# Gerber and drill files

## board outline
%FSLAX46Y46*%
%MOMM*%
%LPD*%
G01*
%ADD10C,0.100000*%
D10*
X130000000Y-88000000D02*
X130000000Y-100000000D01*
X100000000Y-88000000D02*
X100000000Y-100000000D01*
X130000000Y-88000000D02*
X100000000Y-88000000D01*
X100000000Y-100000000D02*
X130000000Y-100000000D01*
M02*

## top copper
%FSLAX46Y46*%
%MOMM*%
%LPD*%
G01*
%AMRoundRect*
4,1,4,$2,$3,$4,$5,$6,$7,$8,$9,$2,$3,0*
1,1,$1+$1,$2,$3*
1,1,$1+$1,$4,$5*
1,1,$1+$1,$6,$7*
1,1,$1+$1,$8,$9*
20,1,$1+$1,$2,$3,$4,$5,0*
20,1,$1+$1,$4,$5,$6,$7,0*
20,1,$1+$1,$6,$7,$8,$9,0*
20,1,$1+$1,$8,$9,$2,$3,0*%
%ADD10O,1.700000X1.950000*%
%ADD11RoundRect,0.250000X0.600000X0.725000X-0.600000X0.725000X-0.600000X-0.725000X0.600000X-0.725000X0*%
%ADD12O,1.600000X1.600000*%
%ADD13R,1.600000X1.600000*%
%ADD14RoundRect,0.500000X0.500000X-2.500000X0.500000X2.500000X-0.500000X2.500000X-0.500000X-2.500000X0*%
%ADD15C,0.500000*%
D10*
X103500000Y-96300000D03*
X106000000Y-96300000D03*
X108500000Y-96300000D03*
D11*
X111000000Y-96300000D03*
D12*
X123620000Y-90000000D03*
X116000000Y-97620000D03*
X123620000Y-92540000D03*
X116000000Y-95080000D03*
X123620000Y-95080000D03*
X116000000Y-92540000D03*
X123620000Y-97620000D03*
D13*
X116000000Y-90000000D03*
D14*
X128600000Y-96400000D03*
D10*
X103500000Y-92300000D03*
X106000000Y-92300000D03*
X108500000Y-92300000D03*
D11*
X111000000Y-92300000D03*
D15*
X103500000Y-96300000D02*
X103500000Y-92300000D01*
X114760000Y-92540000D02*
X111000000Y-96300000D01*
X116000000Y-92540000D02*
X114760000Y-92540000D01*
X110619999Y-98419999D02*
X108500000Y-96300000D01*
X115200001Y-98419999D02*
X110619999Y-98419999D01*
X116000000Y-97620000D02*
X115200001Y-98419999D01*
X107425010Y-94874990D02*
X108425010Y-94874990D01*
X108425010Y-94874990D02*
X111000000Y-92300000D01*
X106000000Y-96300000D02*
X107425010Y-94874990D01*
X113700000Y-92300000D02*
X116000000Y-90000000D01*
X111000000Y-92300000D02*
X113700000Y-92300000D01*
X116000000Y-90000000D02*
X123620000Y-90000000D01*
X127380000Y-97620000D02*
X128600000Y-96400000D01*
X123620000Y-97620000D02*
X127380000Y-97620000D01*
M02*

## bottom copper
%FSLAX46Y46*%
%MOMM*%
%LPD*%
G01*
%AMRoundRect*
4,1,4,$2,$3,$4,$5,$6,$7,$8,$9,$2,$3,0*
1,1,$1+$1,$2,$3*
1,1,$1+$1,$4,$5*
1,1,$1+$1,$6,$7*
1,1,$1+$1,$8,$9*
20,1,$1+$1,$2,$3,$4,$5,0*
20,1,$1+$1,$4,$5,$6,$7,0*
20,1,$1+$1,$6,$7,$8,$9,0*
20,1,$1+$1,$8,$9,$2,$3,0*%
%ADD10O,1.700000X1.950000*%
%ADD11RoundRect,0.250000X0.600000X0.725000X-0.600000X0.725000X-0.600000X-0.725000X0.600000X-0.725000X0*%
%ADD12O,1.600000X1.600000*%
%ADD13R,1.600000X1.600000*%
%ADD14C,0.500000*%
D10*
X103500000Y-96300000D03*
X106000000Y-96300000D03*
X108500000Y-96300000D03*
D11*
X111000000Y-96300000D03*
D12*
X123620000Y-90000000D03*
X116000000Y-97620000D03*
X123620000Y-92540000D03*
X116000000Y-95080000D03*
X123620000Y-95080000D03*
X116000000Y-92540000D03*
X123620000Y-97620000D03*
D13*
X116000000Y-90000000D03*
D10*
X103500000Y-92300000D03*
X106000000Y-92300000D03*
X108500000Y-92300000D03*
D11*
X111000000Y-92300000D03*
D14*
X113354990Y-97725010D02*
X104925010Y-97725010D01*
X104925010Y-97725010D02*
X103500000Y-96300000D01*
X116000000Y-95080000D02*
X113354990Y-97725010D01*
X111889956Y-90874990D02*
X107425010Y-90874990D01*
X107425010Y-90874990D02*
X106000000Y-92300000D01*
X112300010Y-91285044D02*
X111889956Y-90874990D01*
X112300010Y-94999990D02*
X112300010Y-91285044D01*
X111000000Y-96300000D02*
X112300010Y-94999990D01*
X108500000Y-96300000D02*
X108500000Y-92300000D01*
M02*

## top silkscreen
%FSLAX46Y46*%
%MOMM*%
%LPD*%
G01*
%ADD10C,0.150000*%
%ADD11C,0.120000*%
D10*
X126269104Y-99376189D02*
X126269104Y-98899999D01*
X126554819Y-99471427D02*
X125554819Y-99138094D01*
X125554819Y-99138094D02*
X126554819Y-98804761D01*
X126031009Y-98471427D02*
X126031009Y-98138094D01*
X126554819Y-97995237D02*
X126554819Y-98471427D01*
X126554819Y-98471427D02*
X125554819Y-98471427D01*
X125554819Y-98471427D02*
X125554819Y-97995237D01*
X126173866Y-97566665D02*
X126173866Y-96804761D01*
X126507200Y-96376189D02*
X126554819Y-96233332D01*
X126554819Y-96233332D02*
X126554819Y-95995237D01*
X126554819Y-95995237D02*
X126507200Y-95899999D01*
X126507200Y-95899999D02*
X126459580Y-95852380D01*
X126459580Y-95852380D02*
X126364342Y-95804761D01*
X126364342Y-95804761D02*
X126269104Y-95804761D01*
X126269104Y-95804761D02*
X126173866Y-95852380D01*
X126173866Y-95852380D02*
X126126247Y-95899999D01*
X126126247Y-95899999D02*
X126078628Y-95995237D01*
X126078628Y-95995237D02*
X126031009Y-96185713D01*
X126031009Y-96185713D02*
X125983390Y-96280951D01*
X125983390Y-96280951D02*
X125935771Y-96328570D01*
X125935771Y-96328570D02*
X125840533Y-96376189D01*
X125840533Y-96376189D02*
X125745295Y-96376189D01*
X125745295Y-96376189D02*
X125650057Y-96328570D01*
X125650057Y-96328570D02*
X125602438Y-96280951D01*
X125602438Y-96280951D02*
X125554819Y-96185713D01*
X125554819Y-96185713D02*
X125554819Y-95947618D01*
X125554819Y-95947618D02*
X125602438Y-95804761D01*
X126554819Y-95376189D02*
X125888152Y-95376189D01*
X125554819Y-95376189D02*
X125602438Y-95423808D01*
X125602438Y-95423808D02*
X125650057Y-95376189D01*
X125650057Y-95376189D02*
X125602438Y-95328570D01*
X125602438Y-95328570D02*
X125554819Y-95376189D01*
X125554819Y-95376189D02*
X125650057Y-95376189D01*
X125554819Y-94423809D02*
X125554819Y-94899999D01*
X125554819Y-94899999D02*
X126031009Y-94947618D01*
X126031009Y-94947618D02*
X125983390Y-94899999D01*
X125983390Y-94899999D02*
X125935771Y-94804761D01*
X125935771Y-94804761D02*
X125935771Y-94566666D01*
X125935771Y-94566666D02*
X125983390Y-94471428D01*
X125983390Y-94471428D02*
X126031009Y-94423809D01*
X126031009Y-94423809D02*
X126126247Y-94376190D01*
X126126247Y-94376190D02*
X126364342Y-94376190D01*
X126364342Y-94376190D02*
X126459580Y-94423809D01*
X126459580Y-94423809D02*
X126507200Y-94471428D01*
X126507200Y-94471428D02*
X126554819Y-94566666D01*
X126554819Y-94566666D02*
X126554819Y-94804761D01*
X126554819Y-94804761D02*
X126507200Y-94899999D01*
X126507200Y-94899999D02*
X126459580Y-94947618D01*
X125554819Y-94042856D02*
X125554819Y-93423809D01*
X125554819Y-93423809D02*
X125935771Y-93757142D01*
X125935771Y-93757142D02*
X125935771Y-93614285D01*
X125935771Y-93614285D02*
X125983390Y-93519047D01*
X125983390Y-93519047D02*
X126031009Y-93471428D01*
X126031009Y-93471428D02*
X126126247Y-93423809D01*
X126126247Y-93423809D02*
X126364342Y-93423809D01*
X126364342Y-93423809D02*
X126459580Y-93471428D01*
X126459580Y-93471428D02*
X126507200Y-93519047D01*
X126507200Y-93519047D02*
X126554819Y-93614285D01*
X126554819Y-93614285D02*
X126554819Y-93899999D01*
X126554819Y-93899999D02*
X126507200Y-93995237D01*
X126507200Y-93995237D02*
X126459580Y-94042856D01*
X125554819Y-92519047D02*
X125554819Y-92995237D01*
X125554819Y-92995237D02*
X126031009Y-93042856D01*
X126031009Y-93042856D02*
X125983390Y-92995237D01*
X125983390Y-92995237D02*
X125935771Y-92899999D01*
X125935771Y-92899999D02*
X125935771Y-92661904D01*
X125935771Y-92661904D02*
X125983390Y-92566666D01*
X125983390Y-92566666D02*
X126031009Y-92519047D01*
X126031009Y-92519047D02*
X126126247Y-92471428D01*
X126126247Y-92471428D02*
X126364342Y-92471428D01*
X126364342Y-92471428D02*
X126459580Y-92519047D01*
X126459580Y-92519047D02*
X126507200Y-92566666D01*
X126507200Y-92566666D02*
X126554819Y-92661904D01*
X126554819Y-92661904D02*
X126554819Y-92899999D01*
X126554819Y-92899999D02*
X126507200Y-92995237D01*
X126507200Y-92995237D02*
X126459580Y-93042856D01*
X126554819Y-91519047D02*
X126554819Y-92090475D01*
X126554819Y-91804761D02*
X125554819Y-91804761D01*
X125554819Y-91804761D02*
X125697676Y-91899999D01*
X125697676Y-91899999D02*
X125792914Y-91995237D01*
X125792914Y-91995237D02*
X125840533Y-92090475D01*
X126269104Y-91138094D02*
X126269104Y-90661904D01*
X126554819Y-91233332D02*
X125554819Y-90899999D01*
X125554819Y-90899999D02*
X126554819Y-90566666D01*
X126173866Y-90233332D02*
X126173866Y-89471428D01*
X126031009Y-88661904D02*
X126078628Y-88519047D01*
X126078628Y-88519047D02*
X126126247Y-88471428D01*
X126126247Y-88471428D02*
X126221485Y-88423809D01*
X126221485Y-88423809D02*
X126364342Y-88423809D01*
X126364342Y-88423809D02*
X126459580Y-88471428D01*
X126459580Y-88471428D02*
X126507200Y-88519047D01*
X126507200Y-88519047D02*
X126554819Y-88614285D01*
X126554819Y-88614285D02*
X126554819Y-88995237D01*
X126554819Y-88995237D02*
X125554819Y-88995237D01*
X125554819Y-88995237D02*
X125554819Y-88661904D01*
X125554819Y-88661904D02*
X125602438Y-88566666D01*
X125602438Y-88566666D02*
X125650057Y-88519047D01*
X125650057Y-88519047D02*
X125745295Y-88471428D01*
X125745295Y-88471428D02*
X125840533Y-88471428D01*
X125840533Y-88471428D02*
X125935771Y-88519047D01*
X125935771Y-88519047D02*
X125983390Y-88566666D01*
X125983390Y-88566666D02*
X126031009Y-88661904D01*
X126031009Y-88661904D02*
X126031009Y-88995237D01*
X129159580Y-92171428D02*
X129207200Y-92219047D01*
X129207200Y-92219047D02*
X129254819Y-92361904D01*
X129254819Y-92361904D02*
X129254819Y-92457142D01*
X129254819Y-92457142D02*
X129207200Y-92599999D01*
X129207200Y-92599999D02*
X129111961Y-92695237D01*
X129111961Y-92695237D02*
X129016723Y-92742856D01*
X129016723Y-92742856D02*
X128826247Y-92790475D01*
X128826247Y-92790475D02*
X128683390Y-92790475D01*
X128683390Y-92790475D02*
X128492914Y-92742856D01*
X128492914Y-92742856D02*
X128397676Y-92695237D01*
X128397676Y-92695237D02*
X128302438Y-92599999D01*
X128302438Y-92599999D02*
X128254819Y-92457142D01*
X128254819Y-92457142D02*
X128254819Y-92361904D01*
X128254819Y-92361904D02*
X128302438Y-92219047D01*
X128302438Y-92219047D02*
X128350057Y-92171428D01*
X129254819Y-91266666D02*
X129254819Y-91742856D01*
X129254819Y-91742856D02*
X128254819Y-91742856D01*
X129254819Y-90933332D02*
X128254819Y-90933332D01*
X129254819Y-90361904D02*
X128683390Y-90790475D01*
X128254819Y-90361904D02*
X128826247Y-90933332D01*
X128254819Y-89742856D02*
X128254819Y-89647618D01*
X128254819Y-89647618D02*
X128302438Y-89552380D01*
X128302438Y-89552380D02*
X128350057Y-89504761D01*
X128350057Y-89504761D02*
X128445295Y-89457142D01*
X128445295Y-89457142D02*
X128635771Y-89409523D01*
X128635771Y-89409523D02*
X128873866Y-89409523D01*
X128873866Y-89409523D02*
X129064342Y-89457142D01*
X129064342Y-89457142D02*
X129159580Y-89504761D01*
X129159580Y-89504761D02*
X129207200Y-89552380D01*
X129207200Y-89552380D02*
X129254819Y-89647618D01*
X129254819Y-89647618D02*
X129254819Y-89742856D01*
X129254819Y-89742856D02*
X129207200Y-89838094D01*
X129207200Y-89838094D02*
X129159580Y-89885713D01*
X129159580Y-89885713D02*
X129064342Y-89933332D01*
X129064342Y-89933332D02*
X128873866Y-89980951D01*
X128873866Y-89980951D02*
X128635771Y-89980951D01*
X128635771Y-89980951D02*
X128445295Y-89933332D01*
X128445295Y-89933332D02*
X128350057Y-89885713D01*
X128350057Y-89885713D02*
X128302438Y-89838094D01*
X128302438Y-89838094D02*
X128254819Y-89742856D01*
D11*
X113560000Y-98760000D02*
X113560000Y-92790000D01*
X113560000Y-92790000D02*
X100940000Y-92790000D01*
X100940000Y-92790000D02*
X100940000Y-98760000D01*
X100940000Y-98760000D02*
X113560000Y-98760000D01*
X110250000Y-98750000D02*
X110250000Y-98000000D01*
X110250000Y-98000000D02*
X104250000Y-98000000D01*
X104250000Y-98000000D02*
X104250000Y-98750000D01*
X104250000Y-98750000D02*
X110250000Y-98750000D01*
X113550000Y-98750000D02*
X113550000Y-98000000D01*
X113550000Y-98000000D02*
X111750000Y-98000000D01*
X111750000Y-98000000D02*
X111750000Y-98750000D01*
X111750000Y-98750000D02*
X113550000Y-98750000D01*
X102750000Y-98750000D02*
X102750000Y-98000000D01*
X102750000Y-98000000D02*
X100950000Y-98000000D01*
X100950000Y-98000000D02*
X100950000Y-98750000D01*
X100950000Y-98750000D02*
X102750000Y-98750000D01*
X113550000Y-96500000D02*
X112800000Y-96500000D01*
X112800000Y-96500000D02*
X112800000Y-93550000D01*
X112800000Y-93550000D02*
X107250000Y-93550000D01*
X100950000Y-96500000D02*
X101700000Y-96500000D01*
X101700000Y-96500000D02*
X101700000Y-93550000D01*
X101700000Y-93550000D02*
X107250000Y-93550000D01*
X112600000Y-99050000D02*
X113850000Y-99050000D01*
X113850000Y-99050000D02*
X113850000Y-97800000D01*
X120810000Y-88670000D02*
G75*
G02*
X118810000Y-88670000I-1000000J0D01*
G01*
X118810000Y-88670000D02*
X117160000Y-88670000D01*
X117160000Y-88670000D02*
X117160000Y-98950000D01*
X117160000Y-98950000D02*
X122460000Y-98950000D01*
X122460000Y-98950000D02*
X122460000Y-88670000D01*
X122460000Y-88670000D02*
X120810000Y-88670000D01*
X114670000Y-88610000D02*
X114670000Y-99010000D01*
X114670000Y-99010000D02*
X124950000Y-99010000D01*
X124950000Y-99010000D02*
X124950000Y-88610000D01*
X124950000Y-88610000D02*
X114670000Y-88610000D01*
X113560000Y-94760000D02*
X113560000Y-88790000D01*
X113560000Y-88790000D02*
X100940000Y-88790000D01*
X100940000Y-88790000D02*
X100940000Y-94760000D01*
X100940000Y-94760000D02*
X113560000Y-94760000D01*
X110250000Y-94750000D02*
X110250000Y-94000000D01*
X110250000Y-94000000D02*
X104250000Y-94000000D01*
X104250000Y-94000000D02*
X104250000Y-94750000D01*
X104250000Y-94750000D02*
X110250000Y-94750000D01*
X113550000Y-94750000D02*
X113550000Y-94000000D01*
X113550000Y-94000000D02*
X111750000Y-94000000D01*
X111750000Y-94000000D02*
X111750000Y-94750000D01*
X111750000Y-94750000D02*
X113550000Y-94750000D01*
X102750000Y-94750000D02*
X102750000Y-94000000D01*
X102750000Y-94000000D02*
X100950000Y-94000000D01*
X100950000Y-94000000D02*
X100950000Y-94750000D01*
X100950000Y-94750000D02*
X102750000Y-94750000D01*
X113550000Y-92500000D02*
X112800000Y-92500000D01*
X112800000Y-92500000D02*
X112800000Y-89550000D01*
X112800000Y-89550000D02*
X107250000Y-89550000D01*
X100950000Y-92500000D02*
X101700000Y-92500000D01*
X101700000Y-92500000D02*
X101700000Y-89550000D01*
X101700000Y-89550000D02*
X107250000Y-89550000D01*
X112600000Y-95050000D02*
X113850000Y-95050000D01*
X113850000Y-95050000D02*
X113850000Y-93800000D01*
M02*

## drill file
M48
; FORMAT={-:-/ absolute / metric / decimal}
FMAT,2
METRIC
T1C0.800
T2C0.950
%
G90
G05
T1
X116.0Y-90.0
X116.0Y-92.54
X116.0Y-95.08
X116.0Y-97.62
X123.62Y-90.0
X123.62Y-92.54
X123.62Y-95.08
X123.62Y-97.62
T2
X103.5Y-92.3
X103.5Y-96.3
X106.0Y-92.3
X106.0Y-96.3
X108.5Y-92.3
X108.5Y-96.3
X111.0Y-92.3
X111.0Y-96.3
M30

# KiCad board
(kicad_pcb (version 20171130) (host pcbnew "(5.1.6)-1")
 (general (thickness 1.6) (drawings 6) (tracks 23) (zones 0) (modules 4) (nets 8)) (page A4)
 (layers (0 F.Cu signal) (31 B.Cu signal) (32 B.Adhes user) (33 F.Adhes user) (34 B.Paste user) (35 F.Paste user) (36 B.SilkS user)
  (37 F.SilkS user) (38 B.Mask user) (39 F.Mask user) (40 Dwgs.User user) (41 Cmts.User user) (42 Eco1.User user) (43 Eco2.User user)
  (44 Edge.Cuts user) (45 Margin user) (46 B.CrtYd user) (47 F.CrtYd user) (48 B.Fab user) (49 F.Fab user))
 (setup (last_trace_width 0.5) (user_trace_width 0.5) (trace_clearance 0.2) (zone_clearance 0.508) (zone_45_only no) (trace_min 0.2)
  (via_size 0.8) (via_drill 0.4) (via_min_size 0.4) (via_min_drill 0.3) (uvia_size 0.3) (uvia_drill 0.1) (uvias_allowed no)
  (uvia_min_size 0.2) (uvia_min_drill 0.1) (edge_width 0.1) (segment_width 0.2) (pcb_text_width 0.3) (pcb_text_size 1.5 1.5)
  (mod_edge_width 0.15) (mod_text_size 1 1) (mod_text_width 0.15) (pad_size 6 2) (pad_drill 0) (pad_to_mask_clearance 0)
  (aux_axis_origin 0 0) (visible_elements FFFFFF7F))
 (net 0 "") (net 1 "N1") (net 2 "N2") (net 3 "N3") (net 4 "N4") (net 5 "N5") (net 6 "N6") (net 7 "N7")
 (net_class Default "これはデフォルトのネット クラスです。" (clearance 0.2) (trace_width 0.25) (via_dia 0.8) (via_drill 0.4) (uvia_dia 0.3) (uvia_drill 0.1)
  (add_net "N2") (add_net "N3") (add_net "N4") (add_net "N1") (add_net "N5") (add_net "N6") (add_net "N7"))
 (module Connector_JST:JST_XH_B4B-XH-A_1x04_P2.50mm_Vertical (layer F.Cu) (at 111 96.3 180)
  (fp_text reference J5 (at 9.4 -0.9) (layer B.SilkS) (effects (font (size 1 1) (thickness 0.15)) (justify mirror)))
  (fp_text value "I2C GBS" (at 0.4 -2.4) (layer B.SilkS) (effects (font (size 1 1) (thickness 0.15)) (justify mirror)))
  (fp_line (start -2.56 -2.46) (end -2.56 3.51) (layer F.SilkS) (width 0.12))
  (fp_line (start -2.56 3.51) (end 10.06 3.51) (layer F.SilkS) (width 0.12))
  (fp_line (start 10.06 3.51) (end 10.06 -2.46) (layer F.SilkS) (width 0.12))
  (fp_line (start 10.06 -2.46) (end -2.56 -2.46) (layer F.SilkS) (width 0.12))
  (fp_line (start 0.75 -2.45) (end 0.75 -1.7) (layer F.SilkS) (width 0.12))
  (fp_line (start 0.75 -1.7) (end 6.75 -1.7) (layer F.SilkS) (width 0.12))
  (fp_line (start 6.75 -1.7) (end 6.75 -2.45) (layer F.SilkS) (width 0.12))
  (fp_line (start 6.75 -2.45) (end 0.75 -2.45) (layer F.SilkS) (width 0.12))
  (fp_line (start -2.55 -2.45) (end -2.55 -1.7) (layer F.SilkS) (width 0.12))
  (fp_line (start -2.55 -1.7) (end -0.75 -1.7) (layer F.SilkS) (width 0.12))
  (fp_line (start -0.75 -1.7) (end -0.75 -2.45) (layer F.SilkS) (width 0.12))
  (fp_line (start -0.75 -2.45) (end -2.55 -2.45) (layer F.SilkS) (width 0.12))
  (fp_line (start 8.25 -2.45) (end 8.25 -1.7) (layer F.SilkS) (width 0.12))
  (fp_line (start 8.25 -1.7) (end 10.05 -1.7) (layer F.SilkS) (width 0.12))
  (fp_line (start 10.05 -1.7) (end 10.05 -2.45) (layer F.SilkS) (width 0.12))
  (fp_line (start 10.05 -2.45) (end 8.25 -2.45) (layer F.SilkS) (width 0.12))
  (fp_line (start -2.55 -0.2) (end -1.8 -0.2) (layer F.SilkS) (width 0.12))
  (fp_line (start -1.8 -0.2) (end -1.8 2.75) (layer F.SilkS) (width 0.12))
  (fp_line (start -1.8 2.75) (end 3.75 2.75) (layer F.SilkS) (width 0.12))
  (fp_line (start 10.05 -0.2) (end 9.3 -0.2) (layer F.SilkS) (width 0.12))
  (fp_line (start 9.3 -0.2) (end 9.3 2.75) (layer F.SilkS) (width 0.12))
  (fp_line (start 9.3 2.75) (end 3.75 2.75) (layer F.SilkS) (width 0.12))
  (fp_line (start -1.6 -2.75) (end -2.85 -2.75) (layer F.SilkS) (width 0.12))
  (fp_line (start -2.85 -2.75) (end -2.85 -1.5) (layer F.SilkS) (width 0.12))
  (pad 4 thru_hole oval (at 7.5 0 180) (size 1.7 1.95) (drill 0.95) (layers *.Cu *.Mask) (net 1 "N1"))
  (pad 3 thru_hole oval (at 5 0 180) (size 1.7 1.95) (drill 0.95) (layers *.Cu *.Mask) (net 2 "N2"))
  (pad 2 thru_hole oval (at 2.5 0 180) (size 1.7 1.95) (drill 0.95) (layers *.Cu *.Mask) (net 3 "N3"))
  (pad 1 thru_hole roundrect (at 0 0 180) (size 1.7 1.95) (drill 0.95) (layers *.Cu *.Mask) (roundrect_rratio 0.147059) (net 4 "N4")))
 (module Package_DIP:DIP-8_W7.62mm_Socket (layer F.Cu) (at 116 90)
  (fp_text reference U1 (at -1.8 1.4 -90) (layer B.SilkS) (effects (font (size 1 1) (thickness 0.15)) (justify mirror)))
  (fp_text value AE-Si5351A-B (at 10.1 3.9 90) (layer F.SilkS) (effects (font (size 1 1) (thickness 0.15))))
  (fp_arc (start 3.81 -1.33) (end 2.81 -1.33) (angle -180) (layer F.SilkS) (width 0.12))
  (fp_line (start 2.81 -1.33) (end 1.16 -1.33) (layer F.SilkS) (width 0.12))
  (fp_line (start 1.16 -1.33) (end 1.16 8.95) (layer F.SilkS) (width 0.12))
  (fp_line (start 1.16 8.95) (end 6.46 8.95) (layer F.SilkS) (width 0.12))
  (fp_line (start 6.46 8.95) (end 6.46 -1.33) (layer F.SilkS) (width 0.12))
  (fp_line (start 6.46 -1.33) (end 4.81 -1.33) (layer F.SilkS) (width 0.12))
  (fp_line (start -1.33 -1.39) (end -1.33 9.01) (layer F.SilkS) (width 0.12))
  (fp_line (start -1.33 9.01) (end 8.95 9.01) (layer F.SilkS) (width 0.12))
  (fp_line (start 8.95 9.01) (end 8.95 -1.39) (layer F.SilkS) (width 0.12))
  (fp_line (start 8.95 -1.39) (end -1.33 -1.39) (layer F.SilkS) (width 0.12))
  (pad 8 thru_hole oval (at 7.62 0) (size 1.6 1.6) (drill 0.8) (layers *.Cu *.Mask) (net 2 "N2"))
  (pad 4 thru_hole oval (at 0 7.62) (size 1.6 1.6) (drill 0.8) (layers *.Cu *.Mask) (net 3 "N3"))
  (pad 7 thru_hole oval (at 7.62 2.54) (size 1.6 1.6) (drill 0.8) (layers *.Cu *.Mask) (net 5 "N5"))
  (pad 3 thru_hole oval (at 0 5.08) (size 1.6 1.6) (drill 0.8) (layers *.Cu *.Mask) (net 1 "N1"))
  (pad 6 thru_hole oval (at 7.62 5.08) (size 1.6 1.6) (drill 0.8) (layers *.Cu *.Mask) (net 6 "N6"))
  (pad 2 thru_hole oval (at 0 2.54) (size 1.6 1.6) (drill 0.8) (layers *.Cu *.Mask) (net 4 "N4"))
  (pad 5 thru_hole oval (at 7.62 7.62) (size 1.6 1.6) (drill 0.8) (layers *.Cu *.Mask) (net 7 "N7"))
  (pad 1 thru_hole rect (at 0 0) (size 1.6 1.6) (drill 0.8) (layers *.Cu *.Mask) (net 2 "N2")))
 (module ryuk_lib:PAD (layer F.Cu) (at 128.6 96.4 90)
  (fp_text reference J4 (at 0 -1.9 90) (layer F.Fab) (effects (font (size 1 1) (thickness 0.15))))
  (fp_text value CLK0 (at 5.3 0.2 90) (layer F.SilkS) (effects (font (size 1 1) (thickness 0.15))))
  (pad 1 smd roundrect (at 0 0 90) (size 6 2) (layers F.Cu F.Paste F.Mask) (roundrect_rratio 0.25) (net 7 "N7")))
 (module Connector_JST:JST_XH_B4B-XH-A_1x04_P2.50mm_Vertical (layer F.Cu) (at 111 92.3 180)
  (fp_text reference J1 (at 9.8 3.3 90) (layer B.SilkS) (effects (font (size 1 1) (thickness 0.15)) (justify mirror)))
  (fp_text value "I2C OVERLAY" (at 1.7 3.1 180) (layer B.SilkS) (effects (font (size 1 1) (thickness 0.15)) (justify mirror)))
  (fp_line (start -2.56 -2.46) (end -2.56 3.51) (layer F.SilkS) (width 0.12))
  (fp_line (start -2.56 3.51) (end 10.06 3.51) (layer F.SilkS) (width 0.12))
  (fp_line (start 10.06 3.51) (end 10.06 -2.46) (layer F.SilkS) (width 0.12))
  (fp_line (start 10.06 -2.46) (end -2.56 -2.46) (layer F.SilkS) (width 0.12))
  (fp_line (start 0.75 -2.45) (end 0.75 -1.7) (layer F.SilkS) (width 0.12))
  (fp_line (start 0.75 -1.7) (end 6.75 -1.7) (layer F.SilkS) (width 0.12))
  (fp_line (start 6.75 -1.7) (end 6.75 -2.45) (layer F.SilkS) (width 0.12))
  (fp_line (start 6.75 -2.45) (end 0.75 -2.45) (layer F.SilkS) (width 0.12))
  (fp_line (start -2.55 -2.45) (end -2.55 -1.7) (layer F.SilkS) (width 0.12))
  (fp_line (start -2.55 -1.7) (end -0.75 -1.7) (layer F.SilkS) (width 0.12))
  (fp_line (start -0.75 -1.7) (end -0.75 -2.45) (layer F.SilkS) (width 0.12))
  (fp_line (start -0.75 -2.45) (end -2.55 -2.45) (layer F.SilkS) (width 0.12))
  (fp_line (start 8.25 -2.45) (end 8.25 -1.7) (layer F.SilkS) (width 0.12))
  (fp_line (start 8.25 -1.7) (end 10.05 -1.7) (layer F.SilkS) (width 0.12))
  (fp_line (start 10.05 -1.7) (end 10.05 -2.45) (layer F.SilkS) (width 0.12))
  (fp_line (start 10.05 -2.45) (end 8.25 -2.45) (layer F.SilkS) (width 0.12))
  (fp_line (start -2.55 -0.2) (end -1.8 -0.2) (layer F.SilkS) (width 0.12))
  (fp_line (start -1.8 -0.2) (end -1.8 2.75) (layer F.SilkS) (width 0.12))
  (fp_line (start -1.8 2.75) (end 3.75 2.75) (layer F.SilkS) (width 0.12))
  (fp_line (start 10.05 -0.2) (end 9.3 -0.2) (layer F.SilkS) (width 0.12))
  (fp_line (start 9.3 -0.2) (end 9.3 2.75) (layer F.SilkS) (width 0.12))
  (fp_line (start 9.3 2.75) (end 3.75 2.75) (layer F.SilkS) (width 0.12))
  (fp_line (start -1.6 -2.75) (end -2.85 -2.75) (layer F.SilkS) (width 0.12))
  (fp_line (start -2.85 -2.75) (end -2.85 -1.5) (layer F.SilkS) (width 0.12))
  (pad 4 thru_hole oval (at 7.5 0 180) (size 1.7 1.95) (drill 0.95) (layers *.Cu *.Mask) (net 1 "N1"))
  (pad 3 thru_hole oval (at 5 0 180) (size 1.7 1.95) (drill 0.95) (layers *.Cu *.Mask) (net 4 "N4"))
  (pad 2 thru_hole oval (at 2.5 0 180) (size 1.7 1.95) (drill 0.95) (layers *.Cu *.Mask) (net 3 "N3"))
  (pad 1 thru_hole roundrect (at 0 0 180) (size 1.7 1.95) (drill 0.95) (layers *.Cu *.Mask) (roundrect_rratio 0.147059) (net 2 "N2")))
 (gr_line (start 130 88) (end 130 100) (layer Edge.Cuts) (width 0.1))
 (gr_line (start 100 88) (end 100 100) (layer Edge.Cuts) (width 0.1))
 (gr_line (start 130 88) (end 100 88) (layer Edge.Cuts) (width 0.1))
 (gr_line (start 100 100) (end 130 100) (layer Edge.Cuts) (width 0.1))
 (segment (start 103.5 96.3) (end 103.5 92.3) (width 0.5) (layer F.Cu) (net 1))
 (segment (start 113.35499 97.72501) (end 104.92501 97.72501) (width 0.5) (layer B.Cu) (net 1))
 (segment (start 104.92501 97.72501) (end 103.5 96.3) (width 0.5) (layer B.Cu) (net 1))
 (segment (start 116 95.08) (end 113.35499 97.72501) (width 0.5) (layer B.Cu) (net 1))
 (segment (start 114.76 92.54) (end 111 96.3) (width 0.5) (layer F.Cu) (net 4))
 (segment (start 116 92.54) (end 114.76 92.54) (width 0.5) (layer F.Cu) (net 4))
 (segment (start 111.889956 90.87499) (end 107.42501 90.87499) (width 0.5) (layer B.Cu) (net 4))
 (segment (start 107.42501 90.87499) (end 106 92.3) (width 0.5) (layer B.Cu) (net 4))
 (segment (start 112.30001 91.285044) (end 111.889956 90.87499) (width 0.5) (layer B.Cu) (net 4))
 (segment (start 112.30001 94.99999) (end 112.30001 91.285044) (width 0.5) (layer B.Cu) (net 4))
 (segment (start 111 96.3) (end 112.30001 94.99999) (width 0.5) (layer B.Cu) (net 4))
 (segment (start 110.619999 98.419999) (end 108.5 96.3) (width 0.5) (layer F.Cu) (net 3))
 (segment (start 115.200001 98.419999) (end 110.619999 98.419999) (width 0.5) (layer F.Cu) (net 3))
 (segment (start 116 97.62) (end 115.200001 98.419999) (width 0.5) (layer F.Cu) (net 3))
 (segment (start 108.5 96.3) (end 108.5 92.3) (width 0.5) (layer B.Cu) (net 3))
 (segment (start 107.42501 94.87499) (end 108.42501 94.87499) (width 0.5) (layer F.Cu) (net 2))
 (segment (start 108.42501 94.87499) (end 111 92.3) (width 0.5) (layer F.Cu) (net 2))
 (segment (start 106 96.3) (end 107.42501 94.87499) (width 0.5) (layer F.Cu) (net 2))
 (segment (start 113.7 92.3) (end 116 90) (width 0.5) (layer F.Cu) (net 2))
 (segment (start 111 92.3) (end 113.7 92.3) (width 0.5) (layer F.Cu) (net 2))
 (segment (start 116 90) (end 123.62 90) (width 0.5) (layer F.Cu) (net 2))
 (segment (start 127.38 97.62) (end 128.6 96.4) (width 0.5) (layer F.Cu) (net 7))
 (segment (start 123.62 97.62) (end 127.38 97.62) (width 0.5) (layer F.Cu) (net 7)))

